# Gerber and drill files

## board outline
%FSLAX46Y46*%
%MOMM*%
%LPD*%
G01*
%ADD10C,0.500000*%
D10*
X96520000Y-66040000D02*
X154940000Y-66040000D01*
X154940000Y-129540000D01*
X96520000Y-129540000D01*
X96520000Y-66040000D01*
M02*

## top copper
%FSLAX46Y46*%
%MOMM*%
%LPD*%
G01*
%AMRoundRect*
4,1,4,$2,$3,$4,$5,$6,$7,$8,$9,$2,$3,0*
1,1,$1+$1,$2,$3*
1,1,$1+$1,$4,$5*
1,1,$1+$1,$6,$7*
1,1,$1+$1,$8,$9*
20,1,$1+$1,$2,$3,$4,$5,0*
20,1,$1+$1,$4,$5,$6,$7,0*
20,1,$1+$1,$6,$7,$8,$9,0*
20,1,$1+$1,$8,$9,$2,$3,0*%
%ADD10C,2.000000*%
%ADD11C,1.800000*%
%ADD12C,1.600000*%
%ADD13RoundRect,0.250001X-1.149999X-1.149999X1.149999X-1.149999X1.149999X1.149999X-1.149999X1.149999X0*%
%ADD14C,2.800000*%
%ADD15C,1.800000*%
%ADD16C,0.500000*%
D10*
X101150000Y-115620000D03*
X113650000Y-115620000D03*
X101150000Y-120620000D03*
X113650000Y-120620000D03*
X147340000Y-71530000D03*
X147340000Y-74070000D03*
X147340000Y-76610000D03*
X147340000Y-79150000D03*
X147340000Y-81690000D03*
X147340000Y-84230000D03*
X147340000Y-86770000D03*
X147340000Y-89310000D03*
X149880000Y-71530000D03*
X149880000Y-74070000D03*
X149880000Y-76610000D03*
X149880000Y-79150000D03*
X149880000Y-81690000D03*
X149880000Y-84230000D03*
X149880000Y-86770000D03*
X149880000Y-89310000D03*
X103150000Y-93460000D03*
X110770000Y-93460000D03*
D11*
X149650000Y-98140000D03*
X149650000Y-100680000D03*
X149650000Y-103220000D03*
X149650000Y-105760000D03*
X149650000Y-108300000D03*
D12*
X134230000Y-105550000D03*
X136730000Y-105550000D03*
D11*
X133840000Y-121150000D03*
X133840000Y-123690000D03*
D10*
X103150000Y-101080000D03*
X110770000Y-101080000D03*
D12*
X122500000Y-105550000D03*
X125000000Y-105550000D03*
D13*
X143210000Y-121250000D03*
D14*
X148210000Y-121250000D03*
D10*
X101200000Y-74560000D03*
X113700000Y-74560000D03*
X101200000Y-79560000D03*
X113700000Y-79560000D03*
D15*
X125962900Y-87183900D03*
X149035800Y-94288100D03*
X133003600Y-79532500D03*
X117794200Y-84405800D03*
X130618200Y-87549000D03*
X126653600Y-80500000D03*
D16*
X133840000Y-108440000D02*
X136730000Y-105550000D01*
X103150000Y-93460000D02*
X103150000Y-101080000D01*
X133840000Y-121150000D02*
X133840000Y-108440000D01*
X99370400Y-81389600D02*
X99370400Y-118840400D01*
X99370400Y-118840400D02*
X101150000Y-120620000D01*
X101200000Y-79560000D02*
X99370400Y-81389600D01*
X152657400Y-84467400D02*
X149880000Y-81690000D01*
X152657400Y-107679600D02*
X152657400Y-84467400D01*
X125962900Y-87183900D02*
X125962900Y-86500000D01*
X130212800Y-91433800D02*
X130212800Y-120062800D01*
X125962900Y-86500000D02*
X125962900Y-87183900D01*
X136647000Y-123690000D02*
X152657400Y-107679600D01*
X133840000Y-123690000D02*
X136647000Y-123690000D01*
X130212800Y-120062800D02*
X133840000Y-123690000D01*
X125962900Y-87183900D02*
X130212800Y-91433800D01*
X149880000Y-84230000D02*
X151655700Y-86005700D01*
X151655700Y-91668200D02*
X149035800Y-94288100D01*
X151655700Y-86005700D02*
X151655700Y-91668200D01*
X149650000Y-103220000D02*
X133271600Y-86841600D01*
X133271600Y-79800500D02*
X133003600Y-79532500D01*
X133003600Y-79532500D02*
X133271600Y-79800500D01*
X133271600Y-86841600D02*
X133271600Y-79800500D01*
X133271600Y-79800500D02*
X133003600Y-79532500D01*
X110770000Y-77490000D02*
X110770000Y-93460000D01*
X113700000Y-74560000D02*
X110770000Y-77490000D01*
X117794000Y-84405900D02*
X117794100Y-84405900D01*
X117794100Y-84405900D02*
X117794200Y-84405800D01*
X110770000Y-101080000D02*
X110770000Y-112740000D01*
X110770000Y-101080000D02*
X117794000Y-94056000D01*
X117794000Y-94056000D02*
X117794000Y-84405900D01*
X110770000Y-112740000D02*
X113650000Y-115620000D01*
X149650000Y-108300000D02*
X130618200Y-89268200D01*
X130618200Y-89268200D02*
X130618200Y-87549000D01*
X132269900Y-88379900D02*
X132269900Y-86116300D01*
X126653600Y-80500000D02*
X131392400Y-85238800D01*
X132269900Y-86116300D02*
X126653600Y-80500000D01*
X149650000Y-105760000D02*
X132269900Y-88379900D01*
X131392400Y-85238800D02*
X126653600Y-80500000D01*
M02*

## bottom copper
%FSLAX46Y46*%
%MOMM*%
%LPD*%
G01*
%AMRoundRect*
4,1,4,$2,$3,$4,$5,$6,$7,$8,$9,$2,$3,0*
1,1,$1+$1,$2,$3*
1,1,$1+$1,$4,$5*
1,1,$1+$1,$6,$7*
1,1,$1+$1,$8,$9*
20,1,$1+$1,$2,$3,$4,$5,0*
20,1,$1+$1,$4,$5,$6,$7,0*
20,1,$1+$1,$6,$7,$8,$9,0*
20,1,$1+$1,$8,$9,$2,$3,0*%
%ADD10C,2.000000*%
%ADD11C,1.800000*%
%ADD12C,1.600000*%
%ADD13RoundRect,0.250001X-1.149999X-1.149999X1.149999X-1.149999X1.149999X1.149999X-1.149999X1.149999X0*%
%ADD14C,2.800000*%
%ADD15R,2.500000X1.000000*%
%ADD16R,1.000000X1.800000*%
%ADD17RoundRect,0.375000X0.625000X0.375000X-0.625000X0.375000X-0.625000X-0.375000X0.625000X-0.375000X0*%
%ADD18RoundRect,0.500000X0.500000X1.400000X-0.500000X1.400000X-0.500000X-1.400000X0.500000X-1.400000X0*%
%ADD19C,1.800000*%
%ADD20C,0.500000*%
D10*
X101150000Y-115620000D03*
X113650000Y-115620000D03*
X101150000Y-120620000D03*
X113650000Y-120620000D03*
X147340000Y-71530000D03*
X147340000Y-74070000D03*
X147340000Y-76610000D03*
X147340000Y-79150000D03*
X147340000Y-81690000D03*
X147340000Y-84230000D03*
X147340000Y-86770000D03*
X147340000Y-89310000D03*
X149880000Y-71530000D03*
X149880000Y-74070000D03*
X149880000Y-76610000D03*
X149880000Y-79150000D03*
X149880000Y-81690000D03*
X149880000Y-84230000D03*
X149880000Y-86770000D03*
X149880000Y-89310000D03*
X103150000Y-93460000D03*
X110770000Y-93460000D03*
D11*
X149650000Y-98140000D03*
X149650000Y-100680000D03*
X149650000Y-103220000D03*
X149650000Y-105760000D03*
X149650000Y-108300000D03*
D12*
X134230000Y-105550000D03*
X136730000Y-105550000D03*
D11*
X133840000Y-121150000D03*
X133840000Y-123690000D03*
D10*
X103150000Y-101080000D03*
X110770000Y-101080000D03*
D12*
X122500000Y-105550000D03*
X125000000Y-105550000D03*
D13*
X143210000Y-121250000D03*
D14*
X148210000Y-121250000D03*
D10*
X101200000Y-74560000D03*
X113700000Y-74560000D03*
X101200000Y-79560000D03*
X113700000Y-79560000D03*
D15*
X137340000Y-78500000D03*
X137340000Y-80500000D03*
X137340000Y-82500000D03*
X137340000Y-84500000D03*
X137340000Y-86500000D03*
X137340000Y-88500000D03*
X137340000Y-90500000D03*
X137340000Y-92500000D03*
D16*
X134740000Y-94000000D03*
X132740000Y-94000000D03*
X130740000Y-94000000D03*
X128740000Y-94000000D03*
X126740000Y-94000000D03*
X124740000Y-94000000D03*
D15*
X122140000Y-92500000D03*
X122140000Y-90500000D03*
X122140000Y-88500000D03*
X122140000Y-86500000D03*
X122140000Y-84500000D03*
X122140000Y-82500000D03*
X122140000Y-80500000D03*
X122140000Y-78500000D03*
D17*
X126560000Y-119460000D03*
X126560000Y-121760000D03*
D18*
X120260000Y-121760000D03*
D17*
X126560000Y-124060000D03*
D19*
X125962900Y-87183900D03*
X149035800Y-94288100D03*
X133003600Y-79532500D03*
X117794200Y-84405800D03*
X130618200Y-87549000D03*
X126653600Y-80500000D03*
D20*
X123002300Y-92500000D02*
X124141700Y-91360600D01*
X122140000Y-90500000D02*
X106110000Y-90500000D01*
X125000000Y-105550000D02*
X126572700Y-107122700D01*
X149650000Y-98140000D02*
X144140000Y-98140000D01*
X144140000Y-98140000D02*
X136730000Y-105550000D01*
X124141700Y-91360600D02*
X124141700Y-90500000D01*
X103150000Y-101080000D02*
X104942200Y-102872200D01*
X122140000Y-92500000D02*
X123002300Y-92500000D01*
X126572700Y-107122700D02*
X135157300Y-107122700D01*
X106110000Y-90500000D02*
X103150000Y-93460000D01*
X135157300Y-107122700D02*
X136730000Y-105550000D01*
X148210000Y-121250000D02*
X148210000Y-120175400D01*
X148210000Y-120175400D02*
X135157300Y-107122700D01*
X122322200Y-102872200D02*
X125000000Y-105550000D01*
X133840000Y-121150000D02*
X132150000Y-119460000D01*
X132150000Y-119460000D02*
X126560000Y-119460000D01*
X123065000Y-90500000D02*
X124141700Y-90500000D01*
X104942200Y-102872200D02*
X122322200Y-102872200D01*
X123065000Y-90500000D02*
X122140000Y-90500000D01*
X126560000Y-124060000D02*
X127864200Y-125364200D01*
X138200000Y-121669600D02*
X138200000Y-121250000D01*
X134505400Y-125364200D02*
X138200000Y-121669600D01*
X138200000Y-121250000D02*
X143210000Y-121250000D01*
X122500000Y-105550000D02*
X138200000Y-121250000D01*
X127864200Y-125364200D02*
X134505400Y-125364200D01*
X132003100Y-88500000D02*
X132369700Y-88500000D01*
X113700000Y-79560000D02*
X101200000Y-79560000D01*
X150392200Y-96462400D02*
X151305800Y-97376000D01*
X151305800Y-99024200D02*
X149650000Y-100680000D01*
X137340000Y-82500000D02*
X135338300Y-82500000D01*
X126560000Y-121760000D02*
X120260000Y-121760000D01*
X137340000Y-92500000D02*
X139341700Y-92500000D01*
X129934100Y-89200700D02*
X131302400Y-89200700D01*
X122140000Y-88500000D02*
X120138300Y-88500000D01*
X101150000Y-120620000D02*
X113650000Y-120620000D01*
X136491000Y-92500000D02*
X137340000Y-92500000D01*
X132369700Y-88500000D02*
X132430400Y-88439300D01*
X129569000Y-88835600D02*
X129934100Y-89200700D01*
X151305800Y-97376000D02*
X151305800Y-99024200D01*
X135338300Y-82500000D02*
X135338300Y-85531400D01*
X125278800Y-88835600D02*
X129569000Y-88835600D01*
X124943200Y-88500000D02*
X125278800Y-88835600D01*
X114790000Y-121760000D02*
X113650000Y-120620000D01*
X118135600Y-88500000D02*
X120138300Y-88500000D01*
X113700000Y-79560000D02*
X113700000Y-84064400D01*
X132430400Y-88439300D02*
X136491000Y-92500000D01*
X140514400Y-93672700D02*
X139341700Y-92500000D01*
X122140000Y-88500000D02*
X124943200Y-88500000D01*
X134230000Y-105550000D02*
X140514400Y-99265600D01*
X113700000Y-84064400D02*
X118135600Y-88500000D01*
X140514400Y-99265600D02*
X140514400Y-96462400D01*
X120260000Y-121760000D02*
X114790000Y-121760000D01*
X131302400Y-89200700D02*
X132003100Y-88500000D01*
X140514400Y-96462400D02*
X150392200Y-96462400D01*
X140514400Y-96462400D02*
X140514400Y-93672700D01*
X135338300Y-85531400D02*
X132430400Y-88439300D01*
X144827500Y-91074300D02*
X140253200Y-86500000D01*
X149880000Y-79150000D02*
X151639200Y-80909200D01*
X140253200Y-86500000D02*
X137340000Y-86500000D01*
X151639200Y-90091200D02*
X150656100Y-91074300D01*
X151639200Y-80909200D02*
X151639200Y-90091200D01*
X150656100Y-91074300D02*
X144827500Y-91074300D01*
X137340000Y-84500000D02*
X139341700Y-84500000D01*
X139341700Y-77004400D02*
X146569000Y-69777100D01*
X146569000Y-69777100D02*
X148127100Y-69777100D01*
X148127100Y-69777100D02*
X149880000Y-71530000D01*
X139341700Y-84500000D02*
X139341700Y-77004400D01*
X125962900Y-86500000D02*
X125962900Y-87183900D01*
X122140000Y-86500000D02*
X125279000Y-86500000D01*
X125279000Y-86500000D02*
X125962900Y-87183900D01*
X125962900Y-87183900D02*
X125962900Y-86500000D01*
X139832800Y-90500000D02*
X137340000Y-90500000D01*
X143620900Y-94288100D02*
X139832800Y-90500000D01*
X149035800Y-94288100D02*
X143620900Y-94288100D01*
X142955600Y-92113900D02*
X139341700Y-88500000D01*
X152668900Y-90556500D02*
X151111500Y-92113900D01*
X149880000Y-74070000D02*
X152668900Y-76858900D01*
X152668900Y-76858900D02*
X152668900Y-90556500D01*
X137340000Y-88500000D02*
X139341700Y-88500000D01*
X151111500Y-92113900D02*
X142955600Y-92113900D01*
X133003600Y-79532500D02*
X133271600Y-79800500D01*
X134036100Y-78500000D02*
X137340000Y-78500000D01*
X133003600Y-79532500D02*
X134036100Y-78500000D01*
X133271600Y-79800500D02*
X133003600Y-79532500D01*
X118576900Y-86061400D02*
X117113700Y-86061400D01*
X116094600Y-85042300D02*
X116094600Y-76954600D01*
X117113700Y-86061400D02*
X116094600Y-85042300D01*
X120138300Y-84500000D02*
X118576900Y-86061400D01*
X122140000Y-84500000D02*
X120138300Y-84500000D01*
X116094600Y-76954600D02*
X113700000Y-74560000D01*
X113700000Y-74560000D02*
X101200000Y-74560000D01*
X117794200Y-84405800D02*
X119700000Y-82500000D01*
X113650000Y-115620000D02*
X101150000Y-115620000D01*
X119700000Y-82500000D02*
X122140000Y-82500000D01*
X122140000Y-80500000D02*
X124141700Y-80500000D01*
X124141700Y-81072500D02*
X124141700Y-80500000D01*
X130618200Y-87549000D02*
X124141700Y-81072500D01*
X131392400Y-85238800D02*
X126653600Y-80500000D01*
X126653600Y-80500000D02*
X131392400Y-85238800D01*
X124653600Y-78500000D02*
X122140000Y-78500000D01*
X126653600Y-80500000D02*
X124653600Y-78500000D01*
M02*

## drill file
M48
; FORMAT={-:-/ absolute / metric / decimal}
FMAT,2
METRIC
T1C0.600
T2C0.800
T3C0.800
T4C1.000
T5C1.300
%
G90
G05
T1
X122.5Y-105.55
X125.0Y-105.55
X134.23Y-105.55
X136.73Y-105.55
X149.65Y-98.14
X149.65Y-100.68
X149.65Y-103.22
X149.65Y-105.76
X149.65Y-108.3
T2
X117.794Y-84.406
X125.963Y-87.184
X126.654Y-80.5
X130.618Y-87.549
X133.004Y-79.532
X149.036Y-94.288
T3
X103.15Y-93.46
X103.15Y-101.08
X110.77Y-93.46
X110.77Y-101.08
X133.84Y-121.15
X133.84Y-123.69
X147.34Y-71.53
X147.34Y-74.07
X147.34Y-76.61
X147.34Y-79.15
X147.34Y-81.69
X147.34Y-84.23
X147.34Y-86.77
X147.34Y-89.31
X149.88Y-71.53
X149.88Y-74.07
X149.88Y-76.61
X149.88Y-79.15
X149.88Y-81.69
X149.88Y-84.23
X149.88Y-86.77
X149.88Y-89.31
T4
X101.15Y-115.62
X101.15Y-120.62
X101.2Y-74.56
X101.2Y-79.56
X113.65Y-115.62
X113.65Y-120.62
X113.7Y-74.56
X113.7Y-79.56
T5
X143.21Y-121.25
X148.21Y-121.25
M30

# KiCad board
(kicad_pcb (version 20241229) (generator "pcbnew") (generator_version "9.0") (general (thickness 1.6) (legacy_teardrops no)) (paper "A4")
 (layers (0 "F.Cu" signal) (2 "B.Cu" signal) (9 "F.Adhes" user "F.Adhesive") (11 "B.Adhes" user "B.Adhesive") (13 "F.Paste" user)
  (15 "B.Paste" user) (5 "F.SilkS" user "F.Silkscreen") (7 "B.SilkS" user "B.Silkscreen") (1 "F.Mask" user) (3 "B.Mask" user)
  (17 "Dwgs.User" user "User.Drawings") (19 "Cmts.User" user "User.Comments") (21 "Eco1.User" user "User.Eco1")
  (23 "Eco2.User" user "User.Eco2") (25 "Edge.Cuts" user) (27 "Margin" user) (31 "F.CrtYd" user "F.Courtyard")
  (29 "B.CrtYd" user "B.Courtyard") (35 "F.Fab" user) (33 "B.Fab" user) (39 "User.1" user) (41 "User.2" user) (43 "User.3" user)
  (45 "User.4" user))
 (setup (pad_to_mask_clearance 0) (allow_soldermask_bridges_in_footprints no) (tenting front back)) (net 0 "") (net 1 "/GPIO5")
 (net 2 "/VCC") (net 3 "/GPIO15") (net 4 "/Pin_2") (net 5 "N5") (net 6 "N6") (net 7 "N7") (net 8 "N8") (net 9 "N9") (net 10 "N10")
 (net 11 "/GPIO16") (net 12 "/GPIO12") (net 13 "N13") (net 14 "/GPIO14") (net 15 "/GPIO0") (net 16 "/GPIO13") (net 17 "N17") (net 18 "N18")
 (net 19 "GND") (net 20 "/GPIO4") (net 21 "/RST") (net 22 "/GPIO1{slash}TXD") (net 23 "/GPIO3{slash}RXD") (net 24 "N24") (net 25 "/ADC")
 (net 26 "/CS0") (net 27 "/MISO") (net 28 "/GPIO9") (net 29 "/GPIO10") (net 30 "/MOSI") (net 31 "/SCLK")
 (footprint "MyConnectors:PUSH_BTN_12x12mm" (layer "F.Cu") (at 101.15 115.62)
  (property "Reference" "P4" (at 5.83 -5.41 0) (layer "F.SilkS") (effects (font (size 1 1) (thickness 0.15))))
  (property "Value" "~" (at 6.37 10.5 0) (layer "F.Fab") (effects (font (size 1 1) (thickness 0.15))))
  (pad "1" thru_hole circle (at 0 0) (size 2 2) (drill 1) (layers "*.Cu" "*.Mask") (remove_unused_layers no) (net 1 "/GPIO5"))
  (pad "1" thru_hole circle (at 12.5 0) (size 2 2) (drill 1) (layers "*.Cu" "*.Mask") (remove_unused_layers no) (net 1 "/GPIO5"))
  (pad "2" thru_hole circle (at 0 5) (size 2 2) (drill 1) (layers "*.Cu" "*.Mask") (remove_unused_layers no) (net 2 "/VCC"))
  (pad "2" thru_hole circle (at 12.5 5) (size 2 2) (drill 1) (layers "*.Cu" "*.Mask") (remove_unused_layers no) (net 2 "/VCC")))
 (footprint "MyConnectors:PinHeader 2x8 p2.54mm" (layer "F.Cu") (at 147.34 71.53)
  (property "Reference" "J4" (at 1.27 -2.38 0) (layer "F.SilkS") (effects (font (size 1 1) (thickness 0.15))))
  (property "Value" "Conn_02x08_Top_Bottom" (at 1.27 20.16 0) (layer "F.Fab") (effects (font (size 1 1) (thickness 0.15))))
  (pad "1" thru_hole circle (at 0 0) (size 2 2) (drill 0.8) (layers "*.Cu" "*.Mask") (remove_unused_layers no) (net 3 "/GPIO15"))
  (pad "2" thru_hole circle (at 0 2.54) (size 2 2) (drill 0.8) (layers "*.Cu" "*.Mask") (remove_unused_layers no) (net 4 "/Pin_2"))
  (pad "3" thru_hole circle (at 0 5.08) (size 2 2) (drill 0.8) (layers "*.Cu" "*.Mask") (remove_unused_layers no) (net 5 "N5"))
  (pad "4" thru_hole circle (at 0 7.62) (size 2 2) (drill 0.8) (layers "*.Cu" "*.Mask") (remove_unused_layers no) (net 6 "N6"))
  (pad "5" thru_hole circle (at 0 10.16) (size 2 2) (drill 0.8) (layers "*.Cu" "*.Mask") (remove_unused_layers no) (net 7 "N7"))
  (pad "6" thru_hole circle (at 0 12.7) (size 2 2) (drill 0.8) (layers "*.Cu" "*.Mask") (remove_unused_layers no) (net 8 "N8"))
  (pad "7" thru_hole circle (at 0 15.24) (size 2 2) (drill 0.8) (layers "*.Cu" "*.Mask") (remove_unused_layers no) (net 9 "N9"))
  (pad "8" thru_hole circle (at 0 17.78) (size 2 2) (drill 0.8) (layers "*.Cu" "*.Mask") (remove_unused_layers no) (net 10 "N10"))
  (pad "9" thru_hole circle (at 2.54 0) (size 2 2) (drill 0.8) (layers "*.Cu" "*.Mask") (remove_unused_layers no) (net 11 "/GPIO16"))
  (pad "10" thru_hole circle (at 2.54 2.54) (size 2 2) (drill 0.8) (layers "*.Cu" "*.Mask") (remove_unused_layers no) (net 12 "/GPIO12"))
  (pad "11" thru_hole circle (at 2.54 5.08) (size 2 2) (drill 0.8) (layers "*.Cu" "*.Mask") (remove_unused_layers no) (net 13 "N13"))
  (pad "12" thru_hole circle (at 2.54 7.62) (size 2 2) (drill 0.8) (layers "*.Cu" "*.Mask") (remove_unused_layers no) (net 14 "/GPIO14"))
  (pad "13" thru_hole circle (at 2.54 10.16) (size 2 2) (drill 0.8) (layers "*.Cu" "*.Mask") (remove_unused_layers no) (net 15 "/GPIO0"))
  (pad "14" thru_hole circle (at 2.54 12.7) (size 2 2) (drill 0.8) (layers "*.Cu" "*.Mask") (remove_unused_layers no) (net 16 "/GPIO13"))
  (pad "15" thru_hole circle (at 2.54 15.24) (size 2 2) (drill 0.8) (layers "*.Cu" "*.Mask") (remove_unused_layers no) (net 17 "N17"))
  (pad "16" thru_hole circle (at 2.54 17.78) (size 2 2) (drill 0.8) (layers "*.Cu" "*.Mask") (remove_unused_layers no) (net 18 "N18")))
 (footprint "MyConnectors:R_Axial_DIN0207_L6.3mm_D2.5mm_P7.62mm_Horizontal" (layer "F.Cu") (at 103.15 93.46)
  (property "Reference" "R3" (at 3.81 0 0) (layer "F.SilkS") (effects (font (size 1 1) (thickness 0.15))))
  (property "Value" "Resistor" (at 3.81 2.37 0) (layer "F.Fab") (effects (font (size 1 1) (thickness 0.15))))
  (pad "1" thru_hole circle (at 0 0) (size 2 2) (drill 0.8) (layers "*.Cu" "*.Mask") (remove_unused_layers no) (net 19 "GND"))
  (pad "2" thru_hole circle (at 7.62 0) (size 2 2) (drill 0.8) (layers "*.Cu" "*.Mask") (remove_unused_layers no) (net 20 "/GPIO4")))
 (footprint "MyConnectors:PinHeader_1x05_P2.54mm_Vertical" (layer "F.Cu") (at 149.65 98.14)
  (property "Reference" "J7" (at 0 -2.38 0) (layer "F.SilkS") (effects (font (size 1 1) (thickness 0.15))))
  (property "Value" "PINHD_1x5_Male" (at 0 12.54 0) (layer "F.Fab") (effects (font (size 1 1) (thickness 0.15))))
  (pad "1" thru_hole circle (at 0 0) (size 1.8 1.8) (drill 0.6) (layers "*.Cu" "*.Mask") (remove_unused_layers no) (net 19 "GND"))
  (pad "2" thru_hole circle (at 0 2.54) (size 1.8 1.8) (drill 0.6) (layers "*.Cu" "*.Mask") (remove_unused_layers no) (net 2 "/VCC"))
  (pad "3" thru_hole circle (at 0 5.08) (size 1.8 1.8) (drill 0.6) (layers "*.Cu" "*.Mask") (remove_unused_layers no) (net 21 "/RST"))
  (pad "4" thru_hole circle (at 0 7.62) (size 1.8 1.8) (drill 0.6) (layers "*.Cu" "*.Mask") (remove_unused_layers no)
   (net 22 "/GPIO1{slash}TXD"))
  (pad "5" thru_hole circle (at 0 10.16) (size 1.8 1.8) (drill 0.6) (layers "*.Cu" "*.Mask") (remove_unused_layers no)
   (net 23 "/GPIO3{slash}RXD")))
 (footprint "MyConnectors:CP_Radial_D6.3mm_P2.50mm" (layer "F.Cu") (at 134.23 105.55)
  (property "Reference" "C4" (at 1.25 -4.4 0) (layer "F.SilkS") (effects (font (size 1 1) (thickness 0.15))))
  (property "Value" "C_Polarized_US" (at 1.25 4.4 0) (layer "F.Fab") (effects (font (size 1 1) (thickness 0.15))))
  (pad "1" thru_hole circle (at 0 0) (size 1.6 1.6) (drill 0.6) (layers "*.Cu" "*.Mask") (remove_unused_layers no) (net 2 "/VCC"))
  (pad "2" thru_hole circle (at 2.5 0) (size 1.6 1.6) (drill 0.6) (layers "*.Cu" "*.Mask") (remove_unused_layers no) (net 19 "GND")))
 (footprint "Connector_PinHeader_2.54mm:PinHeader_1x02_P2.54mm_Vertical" (layer "F.Cu") (at 133.84 121.15)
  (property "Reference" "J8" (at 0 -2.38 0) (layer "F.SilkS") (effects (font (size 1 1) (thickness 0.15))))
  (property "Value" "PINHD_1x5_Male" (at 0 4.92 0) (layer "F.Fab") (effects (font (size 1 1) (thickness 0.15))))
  (pad "1" thru_hole circle (at 0 0) (size 1.8 1.8) (drill 0.8) (layers "*.Cu" "*.Mask") (remove_unused_layers no) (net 19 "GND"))
  (pad "2" thru_hole circle (at 0 2.54) (size 1.8 1.8) (drill 0.8) (layers "*.Cu" "*.Mask") (remove_unused_layers no) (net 15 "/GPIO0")))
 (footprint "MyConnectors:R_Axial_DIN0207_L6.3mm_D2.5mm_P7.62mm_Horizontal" (layer "F.Cu") (at 103.15 101.08)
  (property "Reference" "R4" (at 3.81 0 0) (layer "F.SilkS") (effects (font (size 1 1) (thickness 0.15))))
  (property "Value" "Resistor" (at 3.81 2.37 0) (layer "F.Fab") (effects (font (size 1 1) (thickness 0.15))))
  (pad "1" thru_hole circle (at 0 0) (size 2 2) (drill 0.8) (layers "*.Cu" "*.Mask") (remove_unused_layers no) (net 19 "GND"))
  (pad "2" thru_hole circle (at 7.62 0) (size 2 2) (drill 0.8) (layers "*.Cu" "*.Mask") (remove_unused_layers no) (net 1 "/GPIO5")))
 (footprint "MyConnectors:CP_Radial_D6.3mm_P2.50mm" (layer "F.Cu") (at 122.5 105.55)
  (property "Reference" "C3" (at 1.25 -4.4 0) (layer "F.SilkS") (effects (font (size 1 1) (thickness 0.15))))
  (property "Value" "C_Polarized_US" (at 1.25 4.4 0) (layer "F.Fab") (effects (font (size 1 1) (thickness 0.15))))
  (pad "1" thru_hole circle (at 0 0) (size 1.6 1.6) (drill 0.6) (layers "*.Cu" "*.Mask") (remove_unused_layers no) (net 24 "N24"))
  (pad "2" thru_hole circle (at 2.5 0) (size 1.6 1.6) (drill 0.6) (layers "*.Cu" "*.Mask") (remove_unused_layers no) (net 19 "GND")))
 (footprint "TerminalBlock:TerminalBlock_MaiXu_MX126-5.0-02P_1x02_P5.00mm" (layer "F.Cu") (at 143.21 121.25)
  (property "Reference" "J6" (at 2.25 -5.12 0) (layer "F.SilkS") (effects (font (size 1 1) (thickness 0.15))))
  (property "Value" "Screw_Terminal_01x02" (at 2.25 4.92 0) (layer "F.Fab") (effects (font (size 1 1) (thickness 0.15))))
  (pad "1" thru_hole roundrect (at 0 0) (size 2.8 2.8) (drill 1.3) (layers "*.Cu" "*.Mask") (remove_unused_layers no)
   (roundrect_rratio 0.089286) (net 24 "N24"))
  (pad "2" thru_hole circle (at 5 0) (size 2.8 2.8) (drill 1.3) (layers "*.Cu" "*.Mask") (remove_unused_layers no) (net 19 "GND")))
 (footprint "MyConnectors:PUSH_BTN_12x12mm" (layer "F.Cu") (at 101.2 74.56)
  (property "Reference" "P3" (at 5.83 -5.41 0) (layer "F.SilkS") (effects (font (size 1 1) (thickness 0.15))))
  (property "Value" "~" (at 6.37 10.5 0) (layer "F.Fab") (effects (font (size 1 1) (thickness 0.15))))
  (pad "1" thru_hole circle (at 0 0) (size 2 2) (drill 1) (layers "*.Cu" "*.Mask") (remove_unused_layers no) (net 20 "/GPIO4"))
  (pad "1" thru_hole circle (at 12.5 0) (size 2 2) (drill 1) (layers "*.Cu" "*.Mask") (remove_unused_layers no) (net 20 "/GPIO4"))
  (pad "2" thru_hole circle (at 0 5) (size 2 2) (drill 1) (layers "*.Cu" "*.Mask") (remove_unused_layers no) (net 2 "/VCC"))
  (pad "2" thru_hole circle (at 12.5 5) (size 2 2) (drill 1) (layers "*.Cu" "*.Mask") (remove_unused_layers no) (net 2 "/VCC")))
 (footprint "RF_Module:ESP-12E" (layer "B.Cu") (at 129.74 82 180)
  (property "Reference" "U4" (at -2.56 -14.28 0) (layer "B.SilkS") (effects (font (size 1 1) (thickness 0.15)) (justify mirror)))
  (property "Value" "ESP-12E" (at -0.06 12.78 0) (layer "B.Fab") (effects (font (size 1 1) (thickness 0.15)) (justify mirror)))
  (pad "1" smd rect (at -7.6 3.5 180) (size 2.5 1) (layers "B.Cu" "B.Mask" "B.Paste") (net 21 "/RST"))
  (pad "2" smd rect (at -7.6 1.5 180) (size 2.5 1) (layers "B.Cu" "B.Mask" "B.Paste") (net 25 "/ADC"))
  (pad "3" smd rect (at -7.6 -0.5 180) (size 2.5 1) (layers "B.Cu" "B.Mask" "B.Paste") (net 2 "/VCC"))
  (pad "4" smd rect (at -7.6 -2.5 180) (size 2.5 1) (layers "B.Cu" "B.Mask" "B.Paste") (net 11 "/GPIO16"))
  (pad "5" smd rect (at -7.6 -4.5 180) (size 2.5 1) (layers "B.Cu" "B.Mask" "B.Paste") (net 14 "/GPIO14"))
  (pad "6" smd rect (at -7.6 -6.5 180) (size 2.5 1) (layers "B.Cu" "B.Mask" "B.Paste") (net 12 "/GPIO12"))
  (pad "7" smd rect (at -7.6 -8.5 180) (size 2.5 1) (layers "B.Cu" "B.Mask" "B.Paste") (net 16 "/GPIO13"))
  (pad "8" smd rect (at -7.6 -10.5 180) (size 2.5 1) (layers "B.Cu" "B.Mask" "B.Paste") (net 2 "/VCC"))
  (pad "9" smd rect (at -5 -12 180) (size 1 1.8) (layers "B.Cu" "B.Mask" "B.Paste") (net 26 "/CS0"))
  (pad "10" smd rect (at -3 -12 180) (size 1 1.8) (layers "B.Cu" "B.Mask" "B.Paste") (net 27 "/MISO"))
  (pad "11" smd rect (at -1 -12 180) (size 1 1.8) (layers "B.Cu" "B.Mask" "B.Paste") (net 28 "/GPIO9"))
  (pad "12" smd rect (at 1 -12 180) (size 1 1.8) (layers "B.Cu" "B.Mask" "B.Paste") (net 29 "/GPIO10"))
  (pad "13" smd rect (at 3 -12 180) (size 1 1.8) (layers "B.Cu" "B.Mask" "B.Paste") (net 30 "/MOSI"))
  (pad "14" smd rect (at 5 -12 180) (size 1 1.8) (layers "B.Cu" "B.Mask" "B.Paste") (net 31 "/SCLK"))
  (pad "15" smd rect (at 7.6 -10.5 180) (size 2.5 1) (layers "B.Cu" "B.Mask" "B.Paste") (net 19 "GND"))
  (pad "16" smd rect (at 7.6 -8.5 180) (size 2.5 1) (layers "B.Cu" "B.Mask" "B.Paste") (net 19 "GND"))
  (pad "17" smd rect (at 7.6 -6.5 180) (size 2.5 1) (layers "B.Cu" "B.Mask" "B.Paste") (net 2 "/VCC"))
  (pad "18" smd rect (at 7.6 -4.5 180) (size 2.5 1) (layers "B.Cu" "B.Mask" "B.Paste") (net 15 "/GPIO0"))
  (pad "19" smd rect (at 7.6 -2.5 180) (size 2.5 1) (layers "B.Cu" "B.Mask" "B.Paste") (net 20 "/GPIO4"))
  (pad "20" smd rect (at 7.6 -0.5 180) (size 2.5 1) (layers "B.Cu" "B.Mask" "B.Paste") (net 1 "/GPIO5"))
  (pad "21" smd rect (at 7.6 1.5 180) (size 2.5 1) (layers "B.Cu" "B.Mask" "B.Paste") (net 23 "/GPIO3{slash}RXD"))
  (pad "22" smd rect (at 7.6 3.5 180) (size 2.5 1) (layers "B.Cu" "B.Mask" "B.Paste") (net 22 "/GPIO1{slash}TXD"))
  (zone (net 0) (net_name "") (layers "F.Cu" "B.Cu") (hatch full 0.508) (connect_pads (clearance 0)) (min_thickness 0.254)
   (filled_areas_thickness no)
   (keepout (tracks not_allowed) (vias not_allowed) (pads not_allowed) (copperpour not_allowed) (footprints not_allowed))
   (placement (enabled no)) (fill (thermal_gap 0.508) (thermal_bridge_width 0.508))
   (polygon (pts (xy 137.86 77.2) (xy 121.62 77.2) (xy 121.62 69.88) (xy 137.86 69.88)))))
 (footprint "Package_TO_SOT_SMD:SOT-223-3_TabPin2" (layer "B.Cu") (at 123.41 121.76 180)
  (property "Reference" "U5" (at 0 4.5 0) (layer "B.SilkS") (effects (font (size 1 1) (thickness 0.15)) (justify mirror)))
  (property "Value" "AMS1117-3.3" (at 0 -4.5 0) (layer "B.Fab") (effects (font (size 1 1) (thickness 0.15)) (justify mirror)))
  (pad "1" smd roundrect (at -3.15 2.3 180) (size 2 1.5) (layers "B.Cu" "B.Mask" "B.Paste") (roundrect_rratio 0.25) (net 19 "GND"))
  (pad "2" smd roundrect (at -3.15 0 180) (size 2 1.5) (layers "B.Cu" "B.Mask" "B.Paste") (roundrect_rratio 0.25) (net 2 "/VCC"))
  (pad "2" smd roundrect (at 3.15 0 180) (size 2 3.8) (layers "B.Cu" "B.Mask" "B.Paste") (roundrect_rratio 0.25) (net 2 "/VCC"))
  (pad "3" smd roundrect (at -3.15 -2.3 180) (size 2 1.5) (layers "B.Cu" "B.Mask" "B.Paste") (roundrect_rratio 0.25) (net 24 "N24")))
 (gr_rect (start 96.52 66.04) (end 154.94 129.54) (stroke (width 0.5) (type solid)) (fill no) (locked yes) (layer "Edge.Cuts"))
 (segment (start 133.84 108.44) (end 136.73 105.55) (width 0.5) (layer "F.Cu") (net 19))
 (segment (start 103.15 93.46) (end 103.15 101.08) (width 0.5) (layer "F.Cu") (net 19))
 (segment (start 133.84 121.15) (end 133.84 108.44) (width 0.5) (layer "F.Cu") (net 19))
 (segment (start 123.0023 92.5) (end 124.1417 91.3606) (width 0.5) (layer "B.Cu") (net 19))
 (segment (start 122.14 90.5) (end 106.11 90.5) (width 0.5) (layer "B.Cu") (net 19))
 (segment (start 125 105.55) (end 126.5727 107.1227) (width 0.5) (layer "B.Cu") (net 19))
 (segment (start 149.65 98.14) (end 144.14 98.14) (width 0.5) (layer "B.Cu") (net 19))
 (segment (start 144.14 98.14) (end 136.73 105.55) (width 0.5) (layer "B.Cu") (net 19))
 (segment (start 124.1417 91.3606) (end 124.1417 90.5) (width 0.5) (layer "B.Cu") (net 19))
 (segment (start 103.15 101.08) (end 104.9422 102.8722) (width 0.5) (layer "B.Cu") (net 19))
 (segment (start 122.14 92.5) (end 123.0023 92.5) (width 0.5) (layer "B.Cu") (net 19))
 (segment (start 126.5727 107.1227) (end 135.1573 107.1227) (width 0.5) (layer "B.Cu") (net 19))
 (segment (start 106.11 90.5) (end 103.15 93.46) (width 0.5) (layer "B.Cu") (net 19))
 (segment (start 135.1573 107.1227) (end 136.73 105.55) (width 0.5) (layer "B.Cu") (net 19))
 (segment (start 148.21 121.25) (end 148.21 120.1754) (width 0.5) (layer "B.Cu") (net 19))
 (segment (start 148.21 120.1754) (end 135.1573 107.1227) (width 0.5) (layer "B.Cu") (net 19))
 (segment (start 122.3222 102.8722) (end 125 105.55) (width 0.5) (layer "B.Cu") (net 19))
 (segment (start 133.84 121.15) (end 132.15 119.46) (width 0.5) (layer "B.Cu") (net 19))
 (segment (start 132.15 119.46) (end 126.56 119.46) (width 0.5) (layer "B.Cu") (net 19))
 (segment (start 123.065 90.5) (end 124.1417 90.5) (width 0.5) (layer "B.Cu") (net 19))
 (segment (start 104.9422 102.8722) (end 122.3222 102.8722) (width 0.5) (layer "B.Cu") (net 19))
 (segment (start 123.065 90.5) (end 122.14 90.5) (width 0.5) (layer "B.Cu") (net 19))
 (segment (start 126.56 124.06) (end 127.8642 125.3642) (width 0.5) (layer "B.Cu") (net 24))
 (segment (start 138.2 121.6696) (end 138.2 121.25) (width 0.5) (layer "B.Cu") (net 24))
 (segment (start 134.5054 125.3642) (end 138.2 121.6696) (width 0.5) (layer "B.Cu") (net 24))
 (segment (start 138.2 121.25) (end 143.21 121.25) (width 0.5) (layer "B.Cu") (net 24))
 (segment (start 122.5 105.55) (end 138.2 121.25) (width 0.5) (layer "B.Cu") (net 24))
 (segment (start 127.8642 125.3642) (end 134.5054 125.3642) (width 0.5) (layer "B.Cu") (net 24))
 (segment (start 99.3704 81.3896) (end 99.3704 118.8404) (width 0.5) (layer "F.Cu") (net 2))
 (segment (start 99.3704 118.8404) (end 101.15 120.62) (width 0.5) (layer "F.Cu") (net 2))
 (segment (start 101.2 79.56) (end 99.3704 81.3896) (width 0.5) (layer "F.Cu") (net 2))
 (segment (start 132.0031 88.5) (end 132.3697 88.5) (width 0.5) (layer "B.Cu") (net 2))
 (segment (start 113.7 79.56) (end 101.2 79.56) (width 0.5) (layer "B.Cu") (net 2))
 (segment (start 150.3922 96.4624) (end 151.3058 97.376) (width 0.5) (layer "B.Cu") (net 2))
 (segment (start 151.3058 99.0242) (end 149.65 100.68) (width 0.5) (layer "B.Cu") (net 2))
 (segment (start 137.34 82.5) (end 135.3383 82.5) (width 0.5) (layer "B.Cu") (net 2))
 (segment (start 126.56 121.76) (end 120.26 121.76) (width 0.5) (layer "B.Cu") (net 2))
 (segment (start 137.34 92.5) (end 139.3417 92.5) (width 0.5) (layer "B.Cu") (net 2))
 (segment (start 129.9341 89.2007) (end 131.3024 89.2007) (width 0.5) (layer "B.Cu") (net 2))
 (segment (start 122.14 88.5) (end 120.1383 88.5) (width 0.5) (layer "B.Cu") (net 2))
 (segment (start 101.15 120.62) (end 113.65 120.62) (width 0.5) (layer "B.Cu") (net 2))
 (segment (start 136.491 92.5) (end 137.34 92.5) (width 0.5) (layer "B.Cu") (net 2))
 (segment (start 132.3697 88.5) (end 132.4304 88.4393) (width 0.5) (layer "B.Cu") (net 2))
 (segment (start 129.569 88.8356) (end 129.9341 89.2007) (width 0.5) (layer "B.Cu") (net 2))
 (segment (start 151.3058 97.376) (end 151.3058 99.0242) (width 0.5) (layer "B.Cu") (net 2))
 (segment (start 135.3383 82.5) (end 135.3383 85.5314) (width 0.5) (layer "B.Cu") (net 2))
 (segment (start 125.2788 88.8356) (end 129.569 88.8356) (width 0.5) (layer "B.Cu") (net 2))
 (segment (start 124.9432 88.5) (end 125.2788 88.8356) (width 0.5) (layer "B.Cu") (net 2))
 (segment (start 114.79 121.76) (end 113.65 120.62) (width 0.5) (layer "B.Cu") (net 2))
 (segment (start 118.1356 88.5) (end 120.1383 88.5) (width 0.5) (layer "B.Cu") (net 2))
 (segment (start 113.7 79.56) (end 113.7 84.0644) (width 0.5) (layer "B.Cu") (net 2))
 (segment (start 132.4304 88.4393) (end 136.491 92.5) (width 0.5) (layer "B.Cu") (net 2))
 (segment (start 140.5144 93.6727) (end 139.3417 92.5) (width 0.5) (layer "B.Cu") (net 2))
 (segment (start 122.14 88.5) (end 124.9432 88.5) (width 0.5) (layer "B.Cu") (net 2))
 (segment (start 134.23 105.55) (end 140.5144 99.2656) (width 0.5) (layer "B.Cu") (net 2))
 (segment (start 113.7 84.0644) (end 118.1356 88.5) (width 0.5) (layer "B.Cu") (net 2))
 (segment (start 140.5144 99.2656) (end 140.5144 96.4624) (width 0.5) (layer "B.Cu") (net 2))
 (segment (start 120.26 121.76) (end 114.79 121.76) (width 0.5) (layer "B.Cu") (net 2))
 (segment (start 131.3024 89.2007) (end 132.0031 88.5) (width 0.5) (layer "B.Cu") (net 2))
 (segment (start 140.5144 96.4624) (end 150.3922 96.4624) (width 0.5) (layer "B.Cu") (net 2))
 (segment (start 140.5144 96.4624) (end 140.5144 93.6727) (width 0.5) (layer "B.Cu") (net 2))
 (segment (start 135.3383 85.5314) (end 132.4304 88.4393) (width 0.5) (layer "B.Cu") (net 2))
 (segment (start 144.8275 91.0743) (end 140.2532 86.5) (width 0.5) (layer "B.Cu") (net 14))
 (segment (start 149.88 79.15) (end 151.6392 80.9092) (width 0.5) (layer "B.Cu") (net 14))
 (segment (start 140.2532 86.5) (end 137.34 86.5) (width 0.5) (layer "B.Cu") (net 14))
 (segment (start 151.6392 90.0912) (end 150.6561 91.0743) (width 0.5) (layer "B.Cu") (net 14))
 (segment (start 151.6392 80.9092) (end 151.6392 90.0912) (width 0.5) (layer "B.Cu") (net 14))
 (segment (start 150.6561 91.0743) (end 144.8275 91.0743) (width 0.5) (layer "B.Cu") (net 14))
 (segment (start 137.34 84.5) (end 139.3417 84.5) (width 0.5) (layer "B.Cu") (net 11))
 (segment (start 139.3417 77.0044) (end 146.569 69.7771) (width 0.5) (layer "B.Cu") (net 11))
 (segment (start 146.569 69.7771) (end 148.1271 69.7771) (width 0.5) (layer "B.Cu") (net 11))
 (segment (start 148.1271 69.7771) (end 149.88 71.53) (width 0.5) (layer "B.Cu") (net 11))
 (segment (start 139.3417 84.5) (end 139.3417 77.0044) (width 0.5) (layer "B.Cu") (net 11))
 (segment (start 152.6574 84.4674) (end 149.88 81.69) (width 0.5) (layer "F.Cu") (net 15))
 (segment (start 152.6574 107.6796) (end 152.6574 84.4674) (width 0.5) (layer "F.Cu") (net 15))
 (segment (start 125.9629 87.1839) (end 125.9629 86.5) (width 0.5) (layer "F.Cu") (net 15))
 (segment (start 130.2128 91.4338) (end 130.2128 120.0628) (width 0.5) (layer "F.Cu") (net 15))
 (segment (start 125.9629 86.5) (end 125.9629 87.1839) (width 0.5) (layer "F.Cu") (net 15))
 (segment (start 136.647 123.69) (end 152.6574 107.6796) (width 0.5) (layer "F.Cu") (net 15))
 (segment (start 133.84 123.69) (end 136.647 123.69) (width 0.5) (layer "F.Cu") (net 15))
 (segment (start 130.2128 120.0628) (end 133.84 123.69) (width 0.5) (layer "F.Cu") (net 15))
 (segment (start 125.9629 87.1839) (end 130.2128 91.4338) (width 0.5) (layer "F.Cu") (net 15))
 (via (at 125.9629 87.1839) (size 1.8) (drill 0.8) (layers "F.Cu" "B.Cu") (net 15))
 (segment (start 125.9629 86.5) (end 125.9629 87.1839) (width 0.5) (layer "B.Cu") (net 15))
 (segment (start 122.14 86.5) (end 125.279 86.5) (width 0.5) (layer "B.Cu") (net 15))
 (segment (start 125.279 86.5) (end 125.9629 87.1839) (width 0.5) (layer "B.Cu") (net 15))
 (segment (start 125.9629 87.1839) (end 125.9629 86.5) (width 0.5) (layer "B.Cu") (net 15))
 (segment (start 149.88 84.23) (end 151.6557 86.0057) (width 0.5) (layer "F.Cu") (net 16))
 (segment (start 151.6557 91.6682) (end 149.0358 94.2881) (width 0.5) (layer "F.Cu") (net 16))
 (segment (start 151.6557 86.0057) (end 151.6557 91.6682) (width 0.5) (layer "F.Cu") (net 16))
 (via (at 149.0358 94.2881) (size 1.8) (drill 0.8) (layers "F.Cu" "B.Cu") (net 16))
 (segment (start 139.8328 90.5) (end 137.34 90.5) (width 0.5) (layer "B.Cu") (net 16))
 (segment (start 143.6209 94.2881) (end 139.8328 90.5) (width 0.5) (layer "B.Cu") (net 16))
 (segment (start 149.0358 94.2881) (end 143.6209 94.2881) (width 0.5) (layer "B.Cu") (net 16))
 (segment (start 142.9556 92.1139) (end 139.3417 88.5) (width 0.5) (layer "B.Cu") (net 12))
 (segment (start 152.6689 90.5565) (end 151.1115 92.1139) (width 0.5) (layer "B.Cu") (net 12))
 (segment (start 149.88 74.07) (end 152.6689 76.8589) (width 0.5) (layer "B.Cu") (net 12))
 (segment (start 152.6689 76.8589) (end 152.6689 90.5565) (width 0.5) (layer "B.Cu") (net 12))
 (segment (start 137.34 88.5) (end 139.3417 88.5) (width 0.5) (layer "B.Cu") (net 12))
 (segment (start 151.1115 92.1139) (end 142.9556 92.1139) (width 0.5) (layer "B.Cu") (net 12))
 (segment (start 149.65 103.22) (end 133.2716 86.8416) (width 0.5) (layer "F.Cu") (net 21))
 (segment (start 133.2716 79.8005) (end 133.0036 79.5325) (width 0.5) (layer "F.Cu") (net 21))
 (segment (start 133.0036 79.5325) (end 133.2716 79.8005) (width 0.5) (layer "F.Cu") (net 21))
 (segment (start 133.2716 86.8416) (end 133.2716 79.8005) (width 0.5) (layer "F.Cu") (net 21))
 (segment (start 133.2716 79.8005) (end 133.0036 79.5325) (width 0.5) (layer "F.Cu") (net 21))
 (via (at 133.0036 79.5325) (size 1.8) (drill 0.8) (layers "F.Cu" "B.Cu") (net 21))
 (segment (start 133.0036 79.5325) (end 133.2716 79.8005) (width 0.5) (layer "B.Cu") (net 21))
 (segment (start 134.0361 78.5) (end 137.34 78.5) (width 0.5) (layer "B.Cu") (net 21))
 (segment (start 133.0036 79.5325) (end 134.0361 78.5) (width 0.5) (layer "B.Cu") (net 21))
 (segment (start 133.2716 79.8005) (end 133.0036 79.5325) (width 0.5) (layer "B.Cu") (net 21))
 (segment (start 110.77 77.49) (end 110.77 93.46) (width 0.5) (layer "F.Cu") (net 20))
 (segment (start 113.7 74.56) (end 110.77 77.49) (width 0.5) (layer "F.Cu") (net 20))
 (segment (start 118.5769 86.0614) (end 117.1137 86.0614) (width 0.5) (layer "B.Cu") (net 20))
 (segment (start 116.0946 85.0423) (end 116.0946 76.9546) (width 0.5) (layer "B.Cu") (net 20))
 (segment (start 117.1137 86.0614) (end 116.0946 85.0423) (width 0.5) (layer "B.Cu") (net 20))
 (segment (start 120.1383 84.5) (end 118.5769 86.0614) (width 0.5) (layer "B.Cu") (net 20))
 (segment (start 122.14 84.5) (end 120.1383 84.5) (width 0.5) (layer "B.Cu") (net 20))
 (segment (start 116.0946 76.9546) (end 113.7 74.56) (width 0.5) (layer "B.Cu") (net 20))
 (segment (start 113.7 74.56) (end 101.2 74.56) (width 0.5) (layer "B.Cu") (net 20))
 (segment (start 117.794 84.4059) (end 117.7941 84.4059) (width 0.5) (layer "F.Cu") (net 1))
 (segment (start 117.7941 84.4059) (end 117.7942 84.4058) (width 0.5) (layer "F.Cu") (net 1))
 (segment (start 110.77 101.08) (end 110.77 112.74) (width 0.5) (layer "F.Cu") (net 1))
 (segment (start 110.77 101.08) (end 117.794 94.056) (width 0.5) (layer "F.Cu") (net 1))
 (segment (start 117.794 94.056) (end 117.794 84.4059) (width 0.5) (layer "F.Cu") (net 1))
 (segment (start 110.77 112.74) (end 113.65 115.62) (width 0.5) (layer "F.Cu") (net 1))
 (via (at 117.7942 84.4058) (size 1.8) (drill 0.8) (layers "F.Cu" "B.Cu") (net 1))
 (segment (start 117.7942 84.4058) (end 119.7 82.5) (width 0.5) (layer "B.Cu") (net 1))
 (segment (start 113.65 115.62) (end 101.15 115.62) (width 0.5) (layer "B.Cu") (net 1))
 (segment (start 119.7 82.5) (end 122.14 82.5) (width 0.5) (layer "B.Cu") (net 1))
 (segment (start 149.65 108.3) (end 130.6182 89.2682) (width 0.5) (layer "F.Cu") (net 23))
 (segment (start 130.6182 89.2682) (end 130.6182 87.549) (width 0.5) (layer "F.Cu") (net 23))
 (via (at 130.6182 87.549) (size 1.8) (drill 0.8) (layers "F.Cu" "B.Cu") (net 23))
 (segment (start 122.14 80.5) (end 124.1417 80.5) (width 0.5) (layer "B.Cu") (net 23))
 (segment (start 124.1417 81.0725) (end 124.1417 80.5) (width 0.5) (layer "B.Cu") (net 23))
 (segment (start 130.6182 87.549) (end 124.1417 81.0725) (width 0.5) (layer "B.Cu") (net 23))
 (segment (start 132.2699 88.3799) (end 132.2699 86.1163) (width 0.5) (layer "F.Cu") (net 22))
 (segment (start 126.6536 80.5) (end 131.3924 85.2388) (width 0.5) (layer "F.Cu") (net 22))
 (segment (start 132.2699 86.1163) (end 126.6536 80.5) (width 0.5) (layer "F.Cu") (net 22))
 (segment (start 149.65 105.76) (end 132.2699 88.3799) (width 0.5) (layer "F.Cu") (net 22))
 (segment (start 131.3924 85.2388) (end 126.6536 80.5) (width 0.5) (layer "F.Cu") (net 22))
 (via (at 126.6536 80.5) (size 1.8) (drill 0.8) (layers "F.Cu" "B.Cu") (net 22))
 (segment (start 131.3924 85.2388) (end 126.6536 80.5) (width 0.5) (layer "B.Cu") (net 22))
 (segment (start 126.6536 80.5) (end 131.3924 85.2388) (width 0.5) (layer "B.Cu") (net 22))
 (segment (start 124.6536 78.5) (end 122.14 78.5) (width 0.5) (layer "B.Cu") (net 22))
 (segment (start 126.6536 80.5) (end 124.6536 78.5) (width 0.5) (layer "B.Cu") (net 22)))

